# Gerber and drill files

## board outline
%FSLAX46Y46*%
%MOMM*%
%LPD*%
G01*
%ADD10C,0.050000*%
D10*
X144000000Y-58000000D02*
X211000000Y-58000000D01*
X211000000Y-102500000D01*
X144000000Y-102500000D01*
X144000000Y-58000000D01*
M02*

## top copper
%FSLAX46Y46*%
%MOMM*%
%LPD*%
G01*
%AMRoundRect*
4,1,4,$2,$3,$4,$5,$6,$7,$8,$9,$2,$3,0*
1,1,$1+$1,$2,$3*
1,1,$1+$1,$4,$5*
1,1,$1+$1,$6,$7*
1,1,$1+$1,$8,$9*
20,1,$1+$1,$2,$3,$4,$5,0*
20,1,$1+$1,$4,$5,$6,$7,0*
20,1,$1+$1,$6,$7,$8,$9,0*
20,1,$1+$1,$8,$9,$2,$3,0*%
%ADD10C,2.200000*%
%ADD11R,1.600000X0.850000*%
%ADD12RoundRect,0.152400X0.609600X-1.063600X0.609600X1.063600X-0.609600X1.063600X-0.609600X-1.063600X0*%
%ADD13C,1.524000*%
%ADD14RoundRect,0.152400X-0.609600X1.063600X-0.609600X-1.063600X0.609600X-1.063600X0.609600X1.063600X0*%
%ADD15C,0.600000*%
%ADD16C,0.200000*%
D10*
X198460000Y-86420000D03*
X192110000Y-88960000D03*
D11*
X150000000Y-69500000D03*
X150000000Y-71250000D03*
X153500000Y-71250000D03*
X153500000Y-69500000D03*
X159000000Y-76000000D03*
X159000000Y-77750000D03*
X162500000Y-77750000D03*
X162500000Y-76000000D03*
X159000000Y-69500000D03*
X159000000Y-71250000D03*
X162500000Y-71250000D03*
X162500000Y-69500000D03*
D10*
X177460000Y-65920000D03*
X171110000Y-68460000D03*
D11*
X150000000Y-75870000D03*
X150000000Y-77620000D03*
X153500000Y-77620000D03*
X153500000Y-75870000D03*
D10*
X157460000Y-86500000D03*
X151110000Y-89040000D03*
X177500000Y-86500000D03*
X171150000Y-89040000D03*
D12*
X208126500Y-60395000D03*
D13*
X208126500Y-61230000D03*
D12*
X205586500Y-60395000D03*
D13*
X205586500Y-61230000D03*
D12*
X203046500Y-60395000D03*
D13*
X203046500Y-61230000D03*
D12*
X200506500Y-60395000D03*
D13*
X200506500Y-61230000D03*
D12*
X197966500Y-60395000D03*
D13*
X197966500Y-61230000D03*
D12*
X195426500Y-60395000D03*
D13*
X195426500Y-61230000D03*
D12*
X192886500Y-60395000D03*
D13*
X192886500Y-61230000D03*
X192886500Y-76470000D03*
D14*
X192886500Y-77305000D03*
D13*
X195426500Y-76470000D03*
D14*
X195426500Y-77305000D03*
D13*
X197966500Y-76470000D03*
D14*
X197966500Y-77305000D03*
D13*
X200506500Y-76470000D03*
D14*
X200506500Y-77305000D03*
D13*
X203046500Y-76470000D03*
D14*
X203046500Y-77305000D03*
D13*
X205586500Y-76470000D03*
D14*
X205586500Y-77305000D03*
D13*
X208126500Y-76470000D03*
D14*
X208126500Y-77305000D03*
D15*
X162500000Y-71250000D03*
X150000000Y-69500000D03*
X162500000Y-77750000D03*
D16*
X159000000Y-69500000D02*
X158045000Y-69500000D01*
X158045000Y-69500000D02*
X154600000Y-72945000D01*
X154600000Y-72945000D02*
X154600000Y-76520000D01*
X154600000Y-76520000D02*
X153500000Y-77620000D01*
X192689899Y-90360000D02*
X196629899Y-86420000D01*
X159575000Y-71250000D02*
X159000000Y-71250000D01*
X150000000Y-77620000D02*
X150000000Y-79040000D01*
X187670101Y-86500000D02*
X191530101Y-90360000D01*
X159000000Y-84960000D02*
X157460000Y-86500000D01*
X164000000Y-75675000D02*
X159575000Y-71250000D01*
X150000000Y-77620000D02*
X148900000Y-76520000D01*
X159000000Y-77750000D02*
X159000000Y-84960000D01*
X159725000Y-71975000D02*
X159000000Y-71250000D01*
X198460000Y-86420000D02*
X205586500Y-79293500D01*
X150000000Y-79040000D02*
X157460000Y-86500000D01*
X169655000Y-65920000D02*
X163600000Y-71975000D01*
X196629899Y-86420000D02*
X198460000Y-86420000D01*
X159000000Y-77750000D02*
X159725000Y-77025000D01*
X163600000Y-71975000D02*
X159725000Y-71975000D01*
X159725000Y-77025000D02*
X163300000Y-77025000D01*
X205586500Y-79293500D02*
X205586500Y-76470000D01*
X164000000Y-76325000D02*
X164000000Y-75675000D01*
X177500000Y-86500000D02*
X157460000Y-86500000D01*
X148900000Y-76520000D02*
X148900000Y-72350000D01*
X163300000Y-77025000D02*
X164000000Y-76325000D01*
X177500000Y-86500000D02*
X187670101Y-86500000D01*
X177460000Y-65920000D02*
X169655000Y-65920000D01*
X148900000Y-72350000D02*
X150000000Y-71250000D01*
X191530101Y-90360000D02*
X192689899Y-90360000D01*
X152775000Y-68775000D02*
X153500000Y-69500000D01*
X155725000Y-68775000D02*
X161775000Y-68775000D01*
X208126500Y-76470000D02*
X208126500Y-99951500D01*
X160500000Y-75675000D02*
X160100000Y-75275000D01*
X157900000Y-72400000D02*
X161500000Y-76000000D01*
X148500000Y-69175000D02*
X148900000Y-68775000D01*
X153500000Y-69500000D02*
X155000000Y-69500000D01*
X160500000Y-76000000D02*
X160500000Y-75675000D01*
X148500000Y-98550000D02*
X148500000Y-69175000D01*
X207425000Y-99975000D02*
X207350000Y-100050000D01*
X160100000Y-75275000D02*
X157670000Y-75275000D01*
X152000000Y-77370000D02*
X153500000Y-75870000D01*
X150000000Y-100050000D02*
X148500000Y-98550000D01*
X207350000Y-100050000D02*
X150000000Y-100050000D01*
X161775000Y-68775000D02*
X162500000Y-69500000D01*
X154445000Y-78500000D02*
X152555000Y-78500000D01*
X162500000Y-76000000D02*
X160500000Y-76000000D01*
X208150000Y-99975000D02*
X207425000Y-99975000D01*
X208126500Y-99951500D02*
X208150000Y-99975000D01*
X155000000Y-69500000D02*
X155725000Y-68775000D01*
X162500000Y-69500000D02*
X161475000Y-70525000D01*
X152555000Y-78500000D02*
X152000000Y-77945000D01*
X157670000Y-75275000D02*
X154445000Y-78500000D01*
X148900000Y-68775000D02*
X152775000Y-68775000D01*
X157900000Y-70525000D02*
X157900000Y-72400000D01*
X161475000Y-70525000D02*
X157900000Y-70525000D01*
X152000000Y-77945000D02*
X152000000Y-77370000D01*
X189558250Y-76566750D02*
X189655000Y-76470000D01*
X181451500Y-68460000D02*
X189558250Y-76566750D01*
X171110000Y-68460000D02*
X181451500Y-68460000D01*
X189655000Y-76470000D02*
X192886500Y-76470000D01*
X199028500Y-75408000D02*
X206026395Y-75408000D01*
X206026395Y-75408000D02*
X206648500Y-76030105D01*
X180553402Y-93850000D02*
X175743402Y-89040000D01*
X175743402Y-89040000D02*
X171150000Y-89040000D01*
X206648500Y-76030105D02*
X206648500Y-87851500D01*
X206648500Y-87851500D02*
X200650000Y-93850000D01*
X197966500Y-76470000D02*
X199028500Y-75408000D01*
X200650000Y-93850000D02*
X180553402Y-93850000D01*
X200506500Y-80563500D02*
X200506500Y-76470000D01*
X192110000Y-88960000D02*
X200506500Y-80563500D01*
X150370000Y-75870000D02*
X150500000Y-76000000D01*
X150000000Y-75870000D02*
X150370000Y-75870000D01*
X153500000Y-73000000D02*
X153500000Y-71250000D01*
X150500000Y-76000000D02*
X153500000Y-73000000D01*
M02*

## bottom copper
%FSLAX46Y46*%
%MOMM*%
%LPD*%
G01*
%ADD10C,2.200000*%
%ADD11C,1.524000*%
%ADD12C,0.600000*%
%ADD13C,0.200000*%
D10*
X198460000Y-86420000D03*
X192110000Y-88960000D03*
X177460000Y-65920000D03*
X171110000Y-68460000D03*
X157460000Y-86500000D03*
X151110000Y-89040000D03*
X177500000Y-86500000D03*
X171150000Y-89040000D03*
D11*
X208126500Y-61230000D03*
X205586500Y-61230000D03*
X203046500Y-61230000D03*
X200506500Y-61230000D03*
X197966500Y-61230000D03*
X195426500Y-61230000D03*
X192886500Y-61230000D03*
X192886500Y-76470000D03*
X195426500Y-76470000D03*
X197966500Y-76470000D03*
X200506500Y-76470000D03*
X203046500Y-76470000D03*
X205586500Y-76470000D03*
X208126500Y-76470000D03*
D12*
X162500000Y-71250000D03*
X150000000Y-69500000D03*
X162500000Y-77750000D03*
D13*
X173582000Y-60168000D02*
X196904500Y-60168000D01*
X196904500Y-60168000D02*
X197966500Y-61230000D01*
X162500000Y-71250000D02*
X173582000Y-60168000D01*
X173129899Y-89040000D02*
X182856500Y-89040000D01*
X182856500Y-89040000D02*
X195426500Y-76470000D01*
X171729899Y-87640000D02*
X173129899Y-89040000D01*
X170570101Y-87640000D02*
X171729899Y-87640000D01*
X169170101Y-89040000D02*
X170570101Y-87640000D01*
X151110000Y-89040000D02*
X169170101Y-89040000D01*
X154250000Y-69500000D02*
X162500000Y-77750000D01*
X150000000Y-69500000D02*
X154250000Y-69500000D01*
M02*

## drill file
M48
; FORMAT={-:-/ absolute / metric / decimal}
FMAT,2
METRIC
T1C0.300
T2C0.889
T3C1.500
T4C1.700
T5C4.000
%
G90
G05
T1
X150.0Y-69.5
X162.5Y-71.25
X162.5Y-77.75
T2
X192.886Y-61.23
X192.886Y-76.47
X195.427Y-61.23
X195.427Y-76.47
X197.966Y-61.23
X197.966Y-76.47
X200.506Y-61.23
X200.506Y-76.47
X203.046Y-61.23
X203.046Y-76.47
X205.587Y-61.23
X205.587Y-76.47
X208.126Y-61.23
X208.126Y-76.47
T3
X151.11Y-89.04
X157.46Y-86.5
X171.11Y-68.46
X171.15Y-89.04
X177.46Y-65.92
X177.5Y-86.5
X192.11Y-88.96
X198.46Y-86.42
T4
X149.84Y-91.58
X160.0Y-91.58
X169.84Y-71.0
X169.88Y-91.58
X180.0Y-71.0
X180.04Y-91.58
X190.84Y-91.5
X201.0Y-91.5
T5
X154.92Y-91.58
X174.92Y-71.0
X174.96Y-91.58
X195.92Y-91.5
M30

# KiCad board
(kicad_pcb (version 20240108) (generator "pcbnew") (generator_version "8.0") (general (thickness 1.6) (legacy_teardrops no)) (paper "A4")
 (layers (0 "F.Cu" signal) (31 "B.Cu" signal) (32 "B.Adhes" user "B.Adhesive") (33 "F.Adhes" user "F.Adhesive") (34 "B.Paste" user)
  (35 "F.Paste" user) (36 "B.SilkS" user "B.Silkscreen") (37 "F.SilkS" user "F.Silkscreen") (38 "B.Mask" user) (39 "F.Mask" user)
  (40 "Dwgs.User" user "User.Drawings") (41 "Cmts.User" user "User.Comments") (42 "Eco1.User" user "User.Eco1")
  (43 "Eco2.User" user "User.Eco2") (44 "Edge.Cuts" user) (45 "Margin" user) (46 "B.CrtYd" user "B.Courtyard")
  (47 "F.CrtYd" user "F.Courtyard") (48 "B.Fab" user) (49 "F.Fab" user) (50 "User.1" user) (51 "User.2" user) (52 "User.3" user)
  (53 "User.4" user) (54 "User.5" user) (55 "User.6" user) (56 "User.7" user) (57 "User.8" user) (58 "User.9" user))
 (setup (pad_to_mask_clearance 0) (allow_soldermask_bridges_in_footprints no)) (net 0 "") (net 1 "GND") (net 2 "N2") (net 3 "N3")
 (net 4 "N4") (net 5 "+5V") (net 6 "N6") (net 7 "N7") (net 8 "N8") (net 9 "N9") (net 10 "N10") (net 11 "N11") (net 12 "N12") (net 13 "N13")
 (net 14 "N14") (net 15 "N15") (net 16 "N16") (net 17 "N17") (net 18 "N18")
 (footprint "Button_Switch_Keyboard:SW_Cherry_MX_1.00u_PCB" (layer "F.Cu") (at 198.46 86.42)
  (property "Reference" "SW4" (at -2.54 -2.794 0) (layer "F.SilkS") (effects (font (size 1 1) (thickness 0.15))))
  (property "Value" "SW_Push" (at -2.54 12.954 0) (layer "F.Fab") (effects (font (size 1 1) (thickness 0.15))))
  (pad "" np_thru_hole circle (at -7.62 5.08) (size 1.7 1.7) (drill 1.7) (layers "*.Cu" "*.Mask"))
  (pad "" np_thru_hole circle (at -2.54 5.08) (size 4 4) (drill 4) (layers "*.Cu" "*.Mask"))
  (pad "" np_thru_hole circle (at 2.54 5.08) (size 1.7 1.7) (drill 1.7) (layers "*.Cu" "*.Mask"))
  (pad "1" thru_hole circle (at 0 0) (size 2.2 2.2) (drill 1.5) (layers "*.Cu" "*.Mask") (remove_unused_layers no) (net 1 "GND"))
  (pad "2" thru_hole circle (at -6.35 2.54) (size 2.2 2.2) (drill 1.5) (layers "*.Cu" "*.Mask") (remove_unused_layers no) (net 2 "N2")))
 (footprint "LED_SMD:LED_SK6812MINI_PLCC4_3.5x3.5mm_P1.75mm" (layer "F.Cu") (at 151.75 70.375)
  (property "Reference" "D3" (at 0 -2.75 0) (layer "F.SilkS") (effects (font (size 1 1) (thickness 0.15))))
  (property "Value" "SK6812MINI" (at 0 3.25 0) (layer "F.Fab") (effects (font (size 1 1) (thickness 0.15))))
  (pad "1" smd rect (at -1.75 -0.875) (size 1.6 0.85) (layers "F.Cu" "F.Paste" "F.Mask") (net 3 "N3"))
  (pad "2" smd rect (at -1.75 0.875) (size 1.6 0.85) (layers "F.Cu" "F.Paste" "F.Mask") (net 1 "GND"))
  (pad "3" smd rect (at 1.75 0.875) (size 1.6 0.85) (layers "F.Cu" "F.Paste" "F.Mask") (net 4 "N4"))
  (pad "4" smd rect (at 1.75 -0.875) (size 1.6 0.85) (layers "F.Cu" "F.Paste" "F.Mask") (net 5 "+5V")))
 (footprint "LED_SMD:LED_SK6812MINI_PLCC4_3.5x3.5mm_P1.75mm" (layer "F.Cu") (at 160.75 76.875)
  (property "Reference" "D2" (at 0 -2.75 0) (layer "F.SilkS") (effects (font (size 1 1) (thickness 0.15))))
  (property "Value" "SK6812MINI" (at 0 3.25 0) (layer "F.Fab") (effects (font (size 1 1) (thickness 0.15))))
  (pad "1" smd rect (at -1.75 -0.875) (size 1.6 0.85) (layers "F.Cu" "F.Paste" "F.Mask") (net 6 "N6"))
  (pad "2" smd rect (at -1.75 0.875) (size 1.6 0.85) (layers "F.Cu" "F.Paste" "F.Mask") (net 1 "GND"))
  (pad "3" smd rect (at 1.75 0.875) (size 1.6 0.85) (layers "F.Cu" "F.Paste" "F.Mask") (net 3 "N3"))
  (pad "4" smd rect (at 1.75 -0.875) (size 1.6 0.85) (layers "F.Cu" "F.Paste" "F.Mask") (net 5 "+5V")))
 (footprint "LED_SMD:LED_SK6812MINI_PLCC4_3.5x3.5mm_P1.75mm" (layer "F.Cu") (at 160.75 70.375)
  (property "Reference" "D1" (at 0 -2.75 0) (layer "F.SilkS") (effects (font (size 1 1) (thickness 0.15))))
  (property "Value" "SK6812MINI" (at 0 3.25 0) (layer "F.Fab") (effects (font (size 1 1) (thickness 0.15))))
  (pad "1" smd rect (at -1.75 -0.875) (size 1.6 0.85) (layers "F.Cu" "F.Paste" "F.Mask") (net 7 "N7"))
  (pad "2" smd rect (at -1.75 0.875) (size 1.6 0.85) (layers "F.Cu" "F.Paste" "F.Mask") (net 1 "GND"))
  (pad "3" smd rect (at 1.75 0.875) (size 1.6 0.85) (layers "F.Cu" "F.Paste" "F.Mask") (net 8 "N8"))
  (pad "4" smd rect (at 1.75 -0.875) (size 1.6 0.85) (layers "F.Cu" "F.Paste" "F.Mask") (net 5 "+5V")))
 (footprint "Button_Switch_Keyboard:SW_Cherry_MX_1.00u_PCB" (layer "F.Cu") (at 177.46 65.92)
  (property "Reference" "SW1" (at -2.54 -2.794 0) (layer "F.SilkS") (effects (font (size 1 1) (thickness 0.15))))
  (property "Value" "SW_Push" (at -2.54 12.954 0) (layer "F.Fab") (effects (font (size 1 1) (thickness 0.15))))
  (pad "" np_thru_hole circle (at -7.62 5.08) (size 1.7 1.7) (drill 1.7) (layers "*.Cu" "*.Mask"))
  (pad "" np_thru_hole circle (at -2.54 5.08) (size 4 4) (drill 4) (layers "*.Cu" "*.Mask"))
  (pad "" np_thru_hole circle (at 2.54 5.08) (size 1.7 1.7) (drill 1.7) (layers "*.Cu" "*.Mask"))
  (pad "1" thru_hole circle (at 0 0) (size 2.2 2.2) (drill 1.5) (layers "*.Cu" "*.Mask") (remove_unused_layers no) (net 1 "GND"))
  (pad "2" thru_hole circle (at -6.35 2.54) (size 2.2 2.2) (drill 1.5) (layers "*.Cu" "*.Mask") (remove_unused_layers no) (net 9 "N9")))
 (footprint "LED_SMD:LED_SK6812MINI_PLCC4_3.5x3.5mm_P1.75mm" (layer "F.Cu") (at 151.75 76.745)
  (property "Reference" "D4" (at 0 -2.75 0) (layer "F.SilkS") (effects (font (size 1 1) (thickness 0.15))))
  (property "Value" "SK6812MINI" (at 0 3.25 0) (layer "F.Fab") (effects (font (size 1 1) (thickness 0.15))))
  (pad "1" smd rect (at -1.75 -0.875) (size 1.6 0.85) (layers "F.Cu" "F.Paste" "F.Mask") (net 4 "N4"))
  (pad "2" smd rect (at -1.75 0.875) (size 1.6 0.85) (layers "F.Cu" "F.Paste" "F.Mask") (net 1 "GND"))
  (pad "3" smd rect (at 1.75 0.875) (size 1.6 0.85) (layers "F.Cu" "F.Paste" "F.Mask") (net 7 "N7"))
  (pad "4" smd rect (at 1.75 -0.875) (size 1.6 0.85) (layers "F.Cu" "F.Paste" "F.Mask") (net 5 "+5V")))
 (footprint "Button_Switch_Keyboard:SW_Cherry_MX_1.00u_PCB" (layer "F.Cu") (at 157.46 86.5)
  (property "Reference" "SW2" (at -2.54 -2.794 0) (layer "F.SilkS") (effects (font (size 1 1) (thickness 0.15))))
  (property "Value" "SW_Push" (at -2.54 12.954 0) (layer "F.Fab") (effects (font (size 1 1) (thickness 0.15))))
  (pad "" np_thru_hole circle (at -7.62 5.08) (size 1.7 1.7) (drill 1.7) (layers "*.Cu" "*.Mask"))
  (pad "" np_thru_hole circle (at -2.54 5.08) (size 4 4) (drill 4) (layers "*.Cu" "*.Mask"))
  (pad "" np_thru_hole circle (at 2.54 5.08) (size 1.7 1.7) (drill 1.7) (layers "*.Cu" "*.Mask"))
  (pad "1" thru_hole circle (at 0 0) (size 2.2 2.2) (drill 1.5) (layers "*.Cu" "*.Mask") (remove_unused_layers no) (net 1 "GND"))
  (pad "2" thru_hole circle (at -6.35 2.54) (size 2.2 2.2) (drill 1.5) (layers "*.Cu" "*.Mask") (remove_unused_layers no) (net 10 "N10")))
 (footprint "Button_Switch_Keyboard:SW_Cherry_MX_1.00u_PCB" (layer "F.Cu") (at 177.5 86.5)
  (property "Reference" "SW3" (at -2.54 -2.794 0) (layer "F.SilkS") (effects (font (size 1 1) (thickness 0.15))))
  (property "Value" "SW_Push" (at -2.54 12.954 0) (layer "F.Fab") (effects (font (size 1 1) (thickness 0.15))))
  (pad "" np_thru_hole circle (at -7.62 5.08) (size 1.7 1.7) (drill 1.7) (layers "*.Cu" "*.Mask"))
  (pad "" np_thru_hole circle (at -2.54 5.08) (size 4 4) (drill 4) (layers "*.Cu" "*.Mask"))
  (pad "" np_thru_hole circle (at 2.54 5.08) (size 1.7 1.7) (drill 1.7) (layers "*.Cu" "*.Mask"))
  (pad "1" thru_hole circle (at 0 0) (size 2.2 2.2) (drill 1.5) (layers "*.Cu" "*.Mask") (remove_unused_layers no) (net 1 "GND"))
  (pad "2" thru_hole circle (at -6.35 2.54) (size 2.2 2.2) (drill 1.5) (layers "*.Cu" "*.Mask") (remove_unused_layers no) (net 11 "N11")))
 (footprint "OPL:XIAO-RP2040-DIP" (layer "F.Cu") (at 200.5065 68.85 -90)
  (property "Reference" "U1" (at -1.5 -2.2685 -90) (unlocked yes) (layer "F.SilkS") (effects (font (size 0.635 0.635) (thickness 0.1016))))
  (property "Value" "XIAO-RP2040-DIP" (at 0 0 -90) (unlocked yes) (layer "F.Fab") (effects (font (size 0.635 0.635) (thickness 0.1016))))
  (pad "1" smd roundrect (at -8.455 -7.62 90) (size 2.432 1.524) (layers "F.Cu" "F.Mask") (roundrect_rratio 0.1) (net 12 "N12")
   (thermal_bridge_angle 45))
  (pad "1" thru_hole circle (at -7.62 -7.62 90) (size 1.524 1.524) (drill 0.889) (layers "*.Cu" "*.Mask") (remove_unused_layers no)
   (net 12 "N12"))
  (pad "2" smd roundrect (at -8.455 -5.08 90) (size 2.432 1.524) (layers "F.Cu" "F.Mask") (roundrect_rratio 0.1) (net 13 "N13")
   (thermal_bridge_angle 45))
  (pad "2" thru_hole circle (at -7.62 -5.08 90) (size 1.524 1.524) (drill 0.889) (layers "*.Cu" "*.Mask") (remove_unused_layers no)
   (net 13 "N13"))
  (pad "3" smd roundrect (at -8.455 -2.54 90) (size 2.432 1.524) (layers "F.Cu" "F.Mask") (roundrect_rratio 0.1) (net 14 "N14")
   (thermal_bridge_angle 45))
  (pad "3" thru_hole circle (at -7.62 -2.54 90) (size 1.524 1.524) (drill 0.889) (layers "*.Cu" "*.Mask") (remove_unused_layers no)
   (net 14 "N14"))
  (pad "4" smd roundrect (at -8.455 0 90) (size 2.432 1.524) (layers "F.Cu" "F.Mask") (roundrect_rratio 0.1) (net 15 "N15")
   (thermal_bridge_angle 45))
  (pad "4" thru_hole circle (at -7.62 0 90) (size 1.524 1.524) (drill 0.889) (layers "*.Cu" "*.Mask") (remove_unused_layers no)
   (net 15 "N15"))
  (pad "5" smd roundrect (at -8.455 2.54 90) (size 2.432 1.524) (layers "F.Cu" "F.Mask") (roundrect_rratio 0.1) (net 8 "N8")
   (thermal_bridge_angle 45))
  (pad "5" thru_hole circle (at -7.62 2.54 90) (size 1.524 1.524) (drill 0.889) (layers "*.Cu" "*.Mask") (remove_unused_layers no)
   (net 8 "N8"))
  (pad "6" smd roundrect (at -8.455 5.08 90) (size 2.432 1.524) (layers "F.Cu" "F.Mask") (roundrect_rratio 0.1) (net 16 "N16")
   (thermal_bridge_angle 45))
  (pad "6" thru_hole circle (at -7.62 5.08 90) (size 1.524 1.524) (drill 0.889) (layers "*.Cu" "*.Mask") (remove_unused_layers no)
   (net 16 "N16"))
  (pad "7" smd roundrect (at -8.455 7.62 90) (size 2.432 1.524) (layers "F.Cu" "F.Mask") (roundrect_rratio 0.1) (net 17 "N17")
   (thermal_bridge_angle 45))
  (pad "7" thru_hole circle (at -7.62 7.62 90) (size 1.524 1.524) (drill 0.889) (layers "*.Cu" "*.Mask") (remove_unused_layers no)
   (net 17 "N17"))
  (pad "8" thru_hole circle (at 7.62 7.62 270) (size 1.524 1.524) (drill 0.889) (layers "*.Cu" "*.Mask") (remove_unused_layers no)
   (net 9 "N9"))
  (pad "8" smd roundrect (at 8.455 7.62 270) (size 2.432 1.524) (layers "F.Cu" "F.Mask") (roundrect_rratio 0.1) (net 9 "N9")
   (thermal_bridge_angle 45))
  (pad "9" thru_hole circle (at 7.62 5.08 270) (size 1.524 1.524) (drill 0.889) (layers "*.Cu" "*.Mask") (remove_unused_layers no)
   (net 10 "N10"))
  (pad "9" smd roundrect (at 8.455 5.08 270) (size 2.432 1.524) (layers "F.Cu" "F.Mask") (roundrect_rratio 0.1) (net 10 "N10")
   (thermal_bridge_angle 45))
  (pad "10" thru_hole circle (at 7.62 2.54 270) (size 1.524 1.524) (drill 0.889) (layers "*.Cu" "*.Mask") (remove_unused_layers no)
   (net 11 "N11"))
  (pad "10" smd roundrect (at 8.455 2.54 270) (size 2.432 1.524) (layers "F.Cu" "F.Mask") (roundrect_rratio 0.1) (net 11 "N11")
   (thermal_bridge_angle 45))
  (pad "11" thru_hole circle (at 7.62 0 270) (size 1.524 1.524) (drill 0.889) (layers "*.Cu" "*.Mask") (remove_unused_layers no)
   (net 2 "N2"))
  (pad "11" smd roundrect (at 8.455 0 270) (size 2.432 1.524) (layers "F.Cu" "F.Mask") (roundrect_rratio 0.1) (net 2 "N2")
   (thermal_bridge_angle 45))
  (pad "12" thru_hole circle (at 7.62 -2.54 270) (size 1.524 1.524) (drill 0.889) (layers "*.Cu" "*.Mask") (remove_unused_layers no)
   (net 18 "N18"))
  (pad "12" smd roundrect (at 8.455 -2.54 270) (size 2.432 1.524) (layers "F.Cu" "F.Mask") (roundrect_rratio 0.1) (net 18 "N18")
   (thermal_bridge_angle 45))
  (pad "13" thru_hole circle (at 7.62 -5.08 270) (size 1.524 1.524) (drill 0.889) (layers "*.Cu" "*.Mask") (remove_unused_layers no)
   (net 1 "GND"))
  (pad "13" smd roundrect (at 8.455 -5.08 270) (size 2.432 1.524) (layers "F.Cu" "F.Mask") (roundrect_rratio 0.1) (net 1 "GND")
   (thermal_bridge_angle 45))
  (pad "14" thru_hole circle (at 7.62 -7.62 270) (size 1.524 1.524) (drill 0.889) (layers "*.Cu" "*.Mask") (remove_unused_layers no)
   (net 5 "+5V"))
  (pad "14" smd roundrect (at 8.455 -7.62 270) (size 2.432 1.524) (layers "F.Cu" "F.Mask") (roundrect_rratio 0.1) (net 5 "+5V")
   (thermal_bridge_angle 45)))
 (gr_rect (start 144 58) (end 211 102.5) (stroke (width 0.05) (type default)) (fill none) (layer "Edge.Cuts"))
 (segment (start 159 69.5) (end 158.045 69.5) (width 0.2) (layer "F.Cu") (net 7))
 (segment (start 158.045 69.5) (end 154.6 72.945) (width 0.2) (layer "F.Cu") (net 7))
 (segment (start 154.6 72.945) (end 154.6 76.52) (width 0.2) (layer "F.Cu") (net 7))
 (segment (start 154.6 76.52) (end 153.5 77.62) (width 0.2) (layer "F.Cu") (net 7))
 (segment (start 192.689899 90.36) (end 196.629899 86.42) (width 0.2) (layer "F.Cu") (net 1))
 (segment (start 159.575 71.25) (end 159 71.25) (width 0.2) (layer "F.Cu") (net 1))
 (segment (start 150 77.62) (end 150 79.04) (width 0.2) (layer "F.Cu") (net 1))
 (segment (start 187.670101 86.5) (end 191.530101 90.36) (width 0.2) (layer "F.Cu") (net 1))
 (segment (start 159 84.96) (end 157.46 86.5) (width 0.2) (layer "F.Cu") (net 1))
 (segment (start 164 75.675) (end 159.575 71.25) (width 0.2) (layer "F.Cu") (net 1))
 (segment (start 150 77.62) (end 148.9 76.52) (width 0.2) (layer "F.Cu") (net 1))
 (segment (start 159 77.75) (end 159 84.96) (width 0.2) (layer "F.Cu") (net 1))
 (segment (start 159.725 71.975) (end 159 71.25) (width 0.2) (layer "F.Cu") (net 1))
 (segment (start 198.46 86.42) (end 205.5865 79.2935) (width 0.2) (layer "F.Cu") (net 1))
 (segment (start 150 79.04) (end 157.46 86.5) (width 0.2) (layer "F.Cu") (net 1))
 (segment (start 169.655 65.92) (end 163.6 71.975) (width 0.2) (layer "F.Cu") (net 1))
 (segment (start 196.629899 86.42) (end 198.46 86.42) (width 0.2) (layer "F.Cu") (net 1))
 (segment (start 159 77.75) (end 159.725 77.025) (width 0.2) (layer "F.Cu") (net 1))
 (segment (start 163.6 71.975) (end 159.725 71.975) (width 0.2) (layer "F.Cu") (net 1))
 (segment (start 159.725 77.025) (end 163.3 77.025) (width 0.2) (layer "F.Cu") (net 1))
 (segment (start 205.5865 79.2935) (end 205.5865 76.47) (width 0.2) (layer "F.Cu") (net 1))
 (segment (start 164 76.325) (end 164 75.675) (width 0.2) (layer "F.Cu") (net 1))
 (segment (start 177.5 86.5) (end 157.46 86.5) (width 0.2) (layer "F.Cu") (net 1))
 (segment (start 148.9 76.52) (end 148.9 72.35) (width 0.2) (layer "F.Cu") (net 1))
 (segment (start 163.3 77.025) (end 164 76.325) (width 0.2) (layer "F.Cu") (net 1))
 (segment (start 177.5 86.5) (end 187.670101 86.5) (width 0.2) (layer "F.Cu") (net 1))
 (segment (start 177.46 65.92) (end 169.655 65.92) (width 0.2) (layer "F.Cu") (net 1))
 (segment (start 148.9 72.35) (end 150 71.25) (width 0.2) (layer "F.Cu") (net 1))
 (segment (start 191.530101 90.36) (end 192.689899 90.36) (width 0.2) (layer "F.Cu") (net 1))
 (via (at 162.5 71.25) (size 0.6) (drill 0.3) (layers "F.Cu" "B.Cu") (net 8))
 (segment (start 173.582 60.168) (end 196.9045 60.168) (width 0.2) (layer "B.Cu") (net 8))
 (segment (start 196.9045 60.168) (end 197.9665 61.23) (width 0.2) (layer "B.Cu") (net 8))
 (segment (start 162.5 71.25) (end 173.582 60.168) (width 0.2) (layer "B.Cu") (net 8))
 (segment (start 152.775 68.775) (end 153.5 69.5) (width 0.2) (layer "F.Cu") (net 5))
 (segment (start 155.725 68.775) (end 161.775 68.775) (width 0.2) (layer "F.Cu") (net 5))
 (segment (start 208.1265 76.47) (end 208.1265 99.9515) (width 0.2) (layer "F.Cu") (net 5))
 (segment (start 160.5 75.675) (end 160.1 75.275) (width 0.2) (layer "F.Cu") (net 5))
 (segment (start 157.9 72.4) (end 161.5 76) (width 0.2) (layer "F.Cu") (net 5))
 (segment (start 148.5 69.175) (end 148.9 68.775) (width 0.2) (layer "F.Cu") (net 5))
 (segment (start 153.5 69.5) (end 155 69.5) (width 0.2) (layer "F.Cu") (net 5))
 (segment (start 160.5 76) (end 160.5 75.675) (width 0.2) (layer "F.Cu") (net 5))
 (segment (start 148.5 98.55) (end 148.5 69.175) (width 0.2) (layer "F.Cu") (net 5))
 (segment (start 207.425 99.975) (end 207.35 100.05) (width 0.2) (layer "F.Cu") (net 5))
 (segment (start 160.1 75.275) (end 157.67 75.275) (width 0.2) (layer "F.Cu") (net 5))
 (segment (start 152 77.37) (end 153.5 75.87) (width 0.2) (layer "F.Cu") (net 5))
 (segment (start 150 100.05) (end 148.5 98.55) (width 0.2) (layer "F.Cu") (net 5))
 (segment (start 207.35 100.05) (end 150 100.05) (width 0.2) (layer "F.Cu") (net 5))
 (segment (start 161.775 68.775) (end 162.5 69.5) (width 0.2) (layer "F.Cu") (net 5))
 (segment (start 154.445 78.5) (end 152.555 78.5) (width 0.2) (layer "F.Cu") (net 5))
 (segment (start 162.5 76) (end 160.5 76) (width 0.2) (layer "F.Cu") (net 5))
 (segment (start 208.15 99.975) (end 207.425 99.975) (width 0.2) (layer "F.Cu") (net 5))
 (segment (start 208.1265 99.9515) (end 208.15 99.975) (width 0.2) (layer "F.Cu") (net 5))
 (segment (start 155 69.5) (end 155.725 68.775) (width 0.2) (layer "F.Cu") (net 5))
 (segment (start 162.5 69.5) (end 161.475 70.525) (width 0.2) (layer "F.Cu") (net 5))
 (segment (start 152.555 78.5) (end 152 77.945) (width 0.2) (layer "F.Cu") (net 5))
 (segment (start 157.67 75.275) (end 154.445 78.5) (width 0.2) (layer "F.Cu") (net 5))
 (segment (start 148.9 68.775) (end 152.775 68.775) (width 0.2) (layer "F.Cu") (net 5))
 (segment (start 157.9 70.525) (end 157.9 72.4) (width 0.2) (layer "F.Cu") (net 5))
 (segment (start 161.475 70.525) (end 157.9 70.525) (width 0.2) (layer "F.Cu") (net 5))
 (segment (start 152 77.945) (end 152 77.37) (width 0.2) (layer "F.Cu") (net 5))
 (segment (start 189.55825 76.56675) (end 189.655 76.47) (width 0.2) (layer "F.Cu") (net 9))
 (segment (start 181.4515 68.46) (end 189.55825 76.56675) (width 0.2) (layer "F.Cu") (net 9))
 (segment (start 171.11 68.46) (end 181.4515 68.46) (width 0.2) (layer "F.Cu") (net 9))
 (segment (start 189.655 76.47) (end 192.8865 76.47) (width 0.2) (layer "F.Cu") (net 9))
 (segment (start 173.129899 89.04) (end 182.8565 89.04) (width 0.2) (layer "B.Cu") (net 10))
 (segment (start 182.8565 89.04) (end 195.4265 76.47) (width 0.2) (layer "B.Cu") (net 10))
 (segment (start 171.729899 87.64) (end 173.129899 89.04) (width 0.2) (layer "B.Cu") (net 10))
 (segment (start 170.570101 87.64) (end 171.729899 87.64) (width 0.2) (layer "B.Cu") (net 10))
 (segment (start 169.170101 89.04) (end 170.570101 87.64) (width 0.2) (layer "B.Cu") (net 10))
 (segment (start 151.11 89.04) (end 169.170101 89.04) (width 0.2) (layer "B.Cu") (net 10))
 (segment (start 199.0285 75.408) (end 206.026395 75.408) (width 0.2) (layer "F.Cu") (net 11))
 (segment (start 206.026395 75.408) (end 206.6485 76.030105) (width 0.2) (layer "F.Cu") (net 11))
 (segment (start 180.553402 93.85) (end 175.743402 89.04) (width 0.2) (layer "F.Cu") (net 11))
 (segment (start 175.743402 89.04) (end 171.15 89.04) (width 0.2) (layer "F.Cu") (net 11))
 (segment (start 206.6485 76.030105) (end 206.6485 87.8515) (width 0.2) (layer "F.Cu") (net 11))
 (segment (start 206.6485 87.8515) (end 200.65 93.85) (width 0.2) (layer "F.Cu") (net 11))
 (segment (start 197.9665 76.47) (end 199.0285 75.408) (width 0.2) (layer "F.Cu") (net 11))
 (segment (start 200.65 93.85) (end 180.553402 93.85) (width 0.2) (layer "F.Cu") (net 11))
 (segment (start 200.5065 80.5635) (end 200.5065 76.47) (width 0.2) (layer "F.Cu") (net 2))
 (segment (start 192.11 88.96) (end 200.5065 80.5635) (width 0.2) (layer "F.Cu") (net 2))
 (via (at 150 69.5) (size 0.6) (drill 0.3) (layers "F.Cu" "B.Cu") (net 3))
 (via (at 162.5 77.75) (size 0.6) (drill 0.3) (layers "F.Cu" "B.Cu") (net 3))
 (segment (start 154.25 69.5) (end 162.5 77.75) (width 0.2) (layer "B.Cu") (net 3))
 (segment (start 150 69.5) (end 154.25 69.5) (width 0.2) (layer "B.Cu") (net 3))
 (segment (start 150.37 75.87) (end 150.5 76) (width 0.2) (layer "F.Cu") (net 4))
 (segment (start 150 75.87) (end 150.37 75.87) (width 0.2) (layer "F.Cu") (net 4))
 (segment (start 153.5 73) (end 153.5 71.25) (width 0.2) (layer "F.Cu") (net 4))
 (segment (start 150.5 76) (end 153.5 73) (width 0.2) (layer "F.Cu") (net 4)))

